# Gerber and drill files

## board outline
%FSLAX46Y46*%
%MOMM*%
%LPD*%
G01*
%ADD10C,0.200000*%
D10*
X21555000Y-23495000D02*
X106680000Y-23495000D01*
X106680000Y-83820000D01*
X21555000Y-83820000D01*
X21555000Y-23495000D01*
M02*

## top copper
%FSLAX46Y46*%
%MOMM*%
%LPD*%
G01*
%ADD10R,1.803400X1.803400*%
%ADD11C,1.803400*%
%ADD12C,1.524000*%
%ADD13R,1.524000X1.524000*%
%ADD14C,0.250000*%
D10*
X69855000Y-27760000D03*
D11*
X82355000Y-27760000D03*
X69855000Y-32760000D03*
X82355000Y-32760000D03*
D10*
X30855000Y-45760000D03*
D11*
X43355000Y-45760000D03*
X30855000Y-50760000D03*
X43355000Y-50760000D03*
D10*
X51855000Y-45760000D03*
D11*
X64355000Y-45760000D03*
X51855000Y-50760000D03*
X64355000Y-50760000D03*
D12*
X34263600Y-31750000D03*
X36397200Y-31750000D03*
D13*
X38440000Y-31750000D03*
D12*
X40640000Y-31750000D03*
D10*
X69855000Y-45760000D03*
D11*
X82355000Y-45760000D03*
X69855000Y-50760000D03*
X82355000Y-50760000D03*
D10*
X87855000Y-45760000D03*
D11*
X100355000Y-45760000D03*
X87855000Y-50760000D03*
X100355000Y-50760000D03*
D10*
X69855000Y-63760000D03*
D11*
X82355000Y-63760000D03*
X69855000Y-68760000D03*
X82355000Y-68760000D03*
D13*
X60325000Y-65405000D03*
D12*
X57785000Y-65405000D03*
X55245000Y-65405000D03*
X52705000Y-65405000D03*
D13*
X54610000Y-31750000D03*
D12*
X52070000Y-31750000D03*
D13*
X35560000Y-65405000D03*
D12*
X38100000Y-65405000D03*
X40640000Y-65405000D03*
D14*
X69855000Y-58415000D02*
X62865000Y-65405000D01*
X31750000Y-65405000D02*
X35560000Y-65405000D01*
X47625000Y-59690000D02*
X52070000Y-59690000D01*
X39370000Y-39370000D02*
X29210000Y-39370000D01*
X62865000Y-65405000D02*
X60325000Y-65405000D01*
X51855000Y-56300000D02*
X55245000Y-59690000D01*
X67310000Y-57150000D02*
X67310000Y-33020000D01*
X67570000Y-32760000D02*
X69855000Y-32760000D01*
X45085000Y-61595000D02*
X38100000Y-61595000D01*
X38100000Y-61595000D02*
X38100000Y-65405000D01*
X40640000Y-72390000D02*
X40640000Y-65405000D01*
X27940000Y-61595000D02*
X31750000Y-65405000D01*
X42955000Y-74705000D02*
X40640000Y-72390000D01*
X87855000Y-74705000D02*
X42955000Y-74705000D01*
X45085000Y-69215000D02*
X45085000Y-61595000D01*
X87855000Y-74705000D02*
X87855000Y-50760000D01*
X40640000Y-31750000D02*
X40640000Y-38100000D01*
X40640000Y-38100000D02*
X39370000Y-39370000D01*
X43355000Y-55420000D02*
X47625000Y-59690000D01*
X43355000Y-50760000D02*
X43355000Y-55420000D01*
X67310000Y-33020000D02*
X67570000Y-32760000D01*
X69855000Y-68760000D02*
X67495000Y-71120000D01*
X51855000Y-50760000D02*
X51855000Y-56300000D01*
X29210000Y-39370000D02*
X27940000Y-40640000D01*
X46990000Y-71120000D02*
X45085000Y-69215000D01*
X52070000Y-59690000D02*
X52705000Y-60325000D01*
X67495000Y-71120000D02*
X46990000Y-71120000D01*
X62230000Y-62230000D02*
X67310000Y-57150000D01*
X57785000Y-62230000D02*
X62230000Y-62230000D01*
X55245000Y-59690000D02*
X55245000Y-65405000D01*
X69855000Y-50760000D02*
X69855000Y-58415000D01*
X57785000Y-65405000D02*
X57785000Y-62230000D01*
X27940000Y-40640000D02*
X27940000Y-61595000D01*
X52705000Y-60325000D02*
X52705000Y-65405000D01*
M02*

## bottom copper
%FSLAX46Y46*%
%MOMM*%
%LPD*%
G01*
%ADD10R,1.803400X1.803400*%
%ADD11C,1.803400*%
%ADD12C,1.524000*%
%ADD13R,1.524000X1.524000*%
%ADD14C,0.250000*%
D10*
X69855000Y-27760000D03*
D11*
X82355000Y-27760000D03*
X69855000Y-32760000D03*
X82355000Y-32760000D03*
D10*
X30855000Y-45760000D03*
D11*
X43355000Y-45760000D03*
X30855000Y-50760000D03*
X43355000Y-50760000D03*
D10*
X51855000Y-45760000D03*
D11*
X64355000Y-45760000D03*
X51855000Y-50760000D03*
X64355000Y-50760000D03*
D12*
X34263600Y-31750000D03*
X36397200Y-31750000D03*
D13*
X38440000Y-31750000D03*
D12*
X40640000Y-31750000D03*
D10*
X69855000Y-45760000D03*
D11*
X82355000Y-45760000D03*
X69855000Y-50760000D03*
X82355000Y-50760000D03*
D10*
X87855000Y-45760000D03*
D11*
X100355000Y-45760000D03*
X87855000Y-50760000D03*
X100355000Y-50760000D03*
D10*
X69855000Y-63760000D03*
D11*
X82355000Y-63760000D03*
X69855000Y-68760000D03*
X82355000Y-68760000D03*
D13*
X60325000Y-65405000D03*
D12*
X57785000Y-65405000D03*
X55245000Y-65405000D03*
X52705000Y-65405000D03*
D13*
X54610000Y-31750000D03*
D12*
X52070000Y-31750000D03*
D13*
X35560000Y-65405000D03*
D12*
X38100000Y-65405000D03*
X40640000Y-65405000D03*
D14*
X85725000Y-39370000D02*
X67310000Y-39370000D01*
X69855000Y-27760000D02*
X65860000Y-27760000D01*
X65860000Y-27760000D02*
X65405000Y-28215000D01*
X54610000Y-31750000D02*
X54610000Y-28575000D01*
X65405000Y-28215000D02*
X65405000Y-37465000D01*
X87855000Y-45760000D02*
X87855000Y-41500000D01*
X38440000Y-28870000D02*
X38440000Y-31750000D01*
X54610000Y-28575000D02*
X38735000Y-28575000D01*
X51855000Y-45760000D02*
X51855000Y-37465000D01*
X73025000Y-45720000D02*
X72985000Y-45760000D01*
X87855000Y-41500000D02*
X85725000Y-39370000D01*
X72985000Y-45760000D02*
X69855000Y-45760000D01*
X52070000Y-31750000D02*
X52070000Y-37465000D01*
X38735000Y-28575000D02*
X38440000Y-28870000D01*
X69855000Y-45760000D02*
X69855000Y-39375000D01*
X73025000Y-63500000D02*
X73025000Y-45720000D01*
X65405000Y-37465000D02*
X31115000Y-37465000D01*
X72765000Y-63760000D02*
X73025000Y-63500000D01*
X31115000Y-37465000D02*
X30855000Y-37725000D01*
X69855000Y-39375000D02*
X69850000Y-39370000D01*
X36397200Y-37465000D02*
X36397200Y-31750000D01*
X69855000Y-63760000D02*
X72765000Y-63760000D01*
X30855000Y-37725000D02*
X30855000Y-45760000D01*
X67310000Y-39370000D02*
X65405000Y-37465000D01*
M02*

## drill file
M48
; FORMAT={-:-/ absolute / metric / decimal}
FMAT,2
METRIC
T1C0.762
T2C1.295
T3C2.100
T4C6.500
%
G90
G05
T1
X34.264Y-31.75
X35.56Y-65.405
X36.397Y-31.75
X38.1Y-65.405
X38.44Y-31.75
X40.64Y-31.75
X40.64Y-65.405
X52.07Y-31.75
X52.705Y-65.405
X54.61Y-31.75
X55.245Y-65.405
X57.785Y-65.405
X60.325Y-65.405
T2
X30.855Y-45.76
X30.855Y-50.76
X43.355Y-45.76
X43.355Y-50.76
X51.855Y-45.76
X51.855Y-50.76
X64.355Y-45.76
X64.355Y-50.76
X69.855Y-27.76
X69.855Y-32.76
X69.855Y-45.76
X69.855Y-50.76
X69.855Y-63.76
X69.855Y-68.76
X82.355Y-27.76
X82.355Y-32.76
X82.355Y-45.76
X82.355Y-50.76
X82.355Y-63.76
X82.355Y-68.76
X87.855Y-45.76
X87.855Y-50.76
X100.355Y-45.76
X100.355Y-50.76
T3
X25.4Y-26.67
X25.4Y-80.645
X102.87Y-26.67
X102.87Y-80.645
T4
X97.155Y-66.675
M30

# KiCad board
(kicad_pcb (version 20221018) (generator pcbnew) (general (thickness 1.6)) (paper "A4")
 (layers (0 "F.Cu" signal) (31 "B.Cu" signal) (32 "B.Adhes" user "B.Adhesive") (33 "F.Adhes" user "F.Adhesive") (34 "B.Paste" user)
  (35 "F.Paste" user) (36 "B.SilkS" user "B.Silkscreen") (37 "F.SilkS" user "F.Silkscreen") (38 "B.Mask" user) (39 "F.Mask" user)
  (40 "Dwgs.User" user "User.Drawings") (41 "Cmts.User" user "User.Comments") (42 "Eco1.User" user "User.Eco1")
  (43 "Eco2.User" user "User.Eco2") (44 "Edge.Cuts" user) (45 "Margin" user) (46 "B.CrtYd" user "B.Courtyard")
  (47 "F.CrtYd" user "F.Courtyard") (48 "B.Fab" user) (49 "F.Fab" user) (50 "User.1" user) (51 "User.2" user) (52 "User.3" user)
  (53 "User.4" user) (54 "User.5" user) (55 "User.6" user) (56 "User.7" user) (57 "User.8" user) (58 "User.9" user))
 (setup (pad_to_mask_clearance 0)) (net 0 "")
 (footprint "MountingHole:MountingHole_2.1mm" (layer "F.Cu") (at 102.87 80.645)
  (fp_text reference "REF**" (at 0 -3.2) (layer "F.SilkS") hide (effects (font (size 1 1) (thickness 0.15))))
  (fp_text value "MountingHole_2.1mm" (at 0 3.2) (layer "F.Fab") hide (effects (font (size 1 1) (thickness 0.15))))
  (pad "" np_thru_hole circle (at 0 0) (size 2.1 2.1) (drill 2.1) (layers "F&B.Cu" "*.Mask")))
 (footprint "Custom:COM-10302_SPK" (layer "F.Cu") (at 69.855 27.76)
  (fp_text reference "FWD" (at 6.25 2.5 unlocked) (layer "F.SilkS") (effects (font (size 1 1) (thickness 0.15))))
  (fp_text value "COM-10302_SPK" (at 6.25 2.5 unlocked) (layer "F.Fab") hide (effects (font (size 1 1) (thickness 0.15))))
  (pad "1" thru_hole rect (at 0 0) (size 1.8034 1.8034) (drill 1.2954) (layers "*.Cu" "*.Mask"))
  (pad "2" thru_hole circle (at 12.5 0) (size 1.8034 1.8034) (drill 1.2954) (layers "*.Cu" "*.Mask"))
  (pad "3" thru_hole circle (at 0 5) (size 1.8034 1.8034) (drill 1.2954) (layers "*.Cu" "*.Mask"))
  (pad "4" thru_hole circle (at 12.5 5) (size 1.8034 1.8034) (drill 1.2954) (layers "*.Cu" "*.Mask")))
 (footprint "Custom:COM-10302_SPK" (layer "F.Cu") (at 30.855 45.76)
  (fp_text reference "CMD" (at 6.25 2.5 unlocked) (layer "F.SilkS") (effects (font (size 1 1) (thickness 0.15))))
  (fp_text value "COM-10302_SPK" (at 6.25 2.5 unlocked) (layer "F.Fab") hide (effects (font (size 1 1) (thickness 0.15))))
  (pad "1" thru_hole rect (at 0 0) (size 1.8034 1.8034) (drill 1.2954) (layers "*.Cu" "*.Mask"))
  (pad "2" thru_hole circle (at 12.5 0) (size 1.8034 1.8034) (drill 1.2954) (layers "*.Cu" "*.Mask"))
  (pad "3" thru_hole circle (at 0 5) (size 1.8034 1.8034) (drill 1.2954) (layers "*.Cu" "*.Mask"))
  (pad "4" thru_hole circle (at 12.5 5) (size 1.8034 1.8034) (drill 1.2954) (layers "*.Cu" "*.Mask")))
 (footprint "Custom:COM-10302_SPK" (layer "F.Cu") (at 51.855 45.76)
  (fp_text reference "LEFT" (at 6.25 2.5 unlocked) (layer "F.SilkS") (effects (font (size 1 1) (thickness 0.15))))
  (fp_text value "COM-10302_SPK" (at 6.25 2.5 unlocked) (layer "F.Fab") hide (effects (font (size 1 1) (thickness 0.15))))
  (pad "1" thru_hole rect (at 0 0) (size 1.8034 1.8034) (drill 1.2954) (layers "*.Cu" "*.Mask"))
  (pad "2" thru_hole circle (at 12.5 0) (size 1.8034 1.8034) (drill 1.2954) (layers "*.Cu" "*.Mask"))
  (pad "3" thru_hole circle (at 0 5) (size 1.8034 1.8034) (drill 1.2954) (layers "*.Cu" "*.Mask"))
  (pad "4" thru_hole circle (at 12.5 5) (size 1.8034 1.8034) (drill 1.2954) (layers "*.Cu" "*.Mask")))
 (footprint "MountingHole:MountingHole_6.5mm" (layer "F.Cu") (at 97.155 66.675)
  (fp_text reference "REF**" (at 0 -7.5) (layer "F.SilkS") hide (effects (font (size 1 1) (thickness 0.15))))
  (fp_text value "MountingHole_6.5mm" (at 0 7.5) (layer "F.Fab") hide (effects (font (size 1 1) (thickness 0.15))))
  (pad "" np_thru_hole circle (at 0 0) (size 6.5 6.5) (drill 6.5) (layers "F&B.Cu" "*.Mask")))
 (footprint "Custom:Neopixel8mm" (layer "F.Cu") (at 35.94 31.75)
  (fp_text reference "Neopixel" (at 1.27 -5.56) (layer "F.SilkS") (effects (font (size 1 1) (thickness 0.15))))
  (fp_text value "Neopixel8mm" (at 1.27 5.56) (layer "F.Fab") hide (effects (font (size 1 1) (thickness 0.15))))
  (pad "1" thru_hole circle (at -1.6764 0) (size 1.524 1.524) (drill 0.762) (layers "*.Cu" "*.Mask"))
  (pad "2" thru_hole circle (at 0.4572 0) (size 1.524 1.524) (drill 0.762) (layers "*.Cu" "*.Mask"))
  (pad "3" thru_hole rect (at 2.5 0) (size 1.524 1.524) (drill 0.762) (layers "*.Cu" "*.Mask"))
  (pad "4" thru_hole circle (at 4.7 0) (size 1.524 1.524) (drill 0.762) (layers "*.Cu" "*.Mask")))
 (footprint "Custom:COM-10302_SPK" (layer "F.Cu") (at 69.855 45.76)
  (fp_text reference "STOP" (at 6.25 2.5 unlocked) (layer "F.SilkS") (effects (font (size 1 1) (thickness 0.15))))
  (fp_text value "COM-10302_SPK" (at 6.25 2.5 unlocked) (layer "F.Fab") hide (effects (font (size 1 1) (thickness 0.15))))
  (pad "1" thru_hole rect (at 0 0) (size 1.8034 1.8034) (drill 1.2954) (layers "*.Cu" "*.Mask"))
  (pad "2" thru_hole circle (at 12.5 0) (size 1.8034 1.8034) (drill 1.2954) (layers "*.Cu" "*.Mask"))
  (pad "3" thru_hole circle (at 0 5) (size 1.8034 1.8034) (drill 1.2954) (layers "*.Cu" "*.Mask"))
  (pad "4" thru_hole circle (at 12.5 5) (size 1.8034 1.8034) (drill 1.2954) (layers "*.Cu" "*.Mask")))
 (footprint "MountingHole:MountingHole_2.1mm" (layer "F.Cu") (at 102.87 26.67)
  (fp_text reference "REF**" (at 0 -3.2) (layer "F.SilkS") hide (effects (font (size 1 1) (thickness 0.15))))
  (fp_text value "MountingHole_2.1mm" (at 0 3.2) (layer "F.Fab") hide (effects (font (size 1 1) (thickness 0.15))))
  (pad "" np_thru_hole circle (at 0 0) (size 2.1 2.1) (drill 2.1) (layers "F&B.Cu" "*.Mask")))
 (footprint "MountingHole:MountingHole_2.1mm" (layer "F.Cu") (at 25.4 80.645)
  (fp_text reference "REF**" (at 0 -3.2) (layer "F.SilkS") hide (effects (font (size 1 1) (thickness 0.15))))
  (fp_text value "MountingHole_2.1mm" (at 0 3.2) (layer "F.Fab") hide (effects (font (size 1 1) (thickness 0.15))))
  (pad "" np_thru_hole circle (at 0 0) (size 2.1 2.1) (drill 2.1) (layers "F&B.Cu" "*.Mask")))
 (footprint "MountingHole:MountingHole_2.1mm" (layer "F.Cu") (at 25.4 26.67)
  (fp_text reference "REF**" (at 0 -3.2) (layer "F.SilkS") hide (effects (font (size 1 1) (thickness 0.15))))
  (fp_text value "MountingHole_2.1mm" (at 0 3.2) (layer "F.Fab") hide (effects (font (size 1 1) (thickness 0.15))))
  (pad "" np_thru_hole circle (at 0 0) (size 2.1 2.1) (drill 2.1) (layers "F&B.Cu" "*.Mask")))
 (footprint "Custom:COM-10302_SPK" (layer "F.Cu") (at 87.855 45.76)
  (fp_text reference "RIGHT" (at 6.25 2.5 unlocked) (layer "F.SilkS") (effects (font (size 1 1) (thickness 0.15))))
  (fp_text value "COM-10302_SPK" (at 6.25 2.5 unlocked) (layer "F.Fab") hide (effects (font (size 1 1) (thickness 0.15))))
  (pad "1" thru_hole rect (at 0 0) (size 1.8034 1.8034) (drill 1.2954) (layers "*.Cu" "*.Mask"))
  (pad "2" thru_hole circle (at 12.5 0) (size 1.8034 1.8034) (drill 1.2954) (layers "*.Cu" "*.Mask"))
  (pad "3" thru_hole circle (at 0 5) (size 1.8034 1.8034) (drill 1.2954) (layers "*.Cu" "*.Mask"))
  (pad "4" thru_hole circle (at 12.5 5) (size 1.8034 1.8034) (drill 1.2954) (layers "*.Cu" "*.Mask")))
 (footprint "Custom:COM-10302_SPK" (layer "F.Cu") (at 69.855 63.76)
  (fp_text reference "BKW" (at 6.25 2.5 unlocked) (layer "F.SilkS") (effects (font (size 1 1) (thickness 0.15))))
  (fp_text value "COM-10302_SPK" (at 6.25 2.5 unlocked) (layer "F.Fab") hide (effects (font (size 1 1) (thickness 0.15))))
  (pad "1" thru_hole rect (at 0 0) (size 1.8034 1.8034) (drill 1.2954) (layers "*.Cu" "*.Mask"))
  (pad "2" thru_hole circle (at 12.5 0) (size 1.8034 1.8034) (drill 1.2954) (layers "*.Cu" "*.Mask"))
  (pad "3" thru_hole circle (at 0 5) (size 1.8034 1.8034) (drill 1.2954) (layers "*.Cu" "*.Mask"))
  (pad "4" thru_hole circle (at 12.5 5) (size 1.8034 1.8034) (drill 1.2954) (layers "*.Cu" "*.Mask")))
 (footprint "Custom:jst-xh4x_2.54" (layer "B.Cu") (at 55.245 67.945 90)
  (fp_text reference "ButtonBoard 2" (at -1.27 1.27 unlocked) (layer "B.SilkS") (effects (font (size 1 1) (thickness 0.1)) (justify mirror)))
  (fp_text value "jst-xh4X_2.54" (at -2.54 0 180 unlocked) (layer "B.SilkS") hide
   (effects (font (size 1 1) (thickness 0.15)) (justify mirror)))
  (pad "1" thru_hole rect (at 2.54 5.08 90) (size 1.524 1.524) (drill 0.762) (layers "*.Cu" "*.Mask"))
  (pad "2" thru_hole circle (at 2.54 2.54 90) (size 1.524 1.524) (drill 0.762) (layers "*.Cu" "*.Mask"))
  (pad "3" thru_hole circle (at 2.54 0 90) (size 1.524 1.524) (drill 0.762) (layers "*.Cu" "*.Mask"))
  (pad "4" thru_hole circle (at 2.54 -2.54 90) (size 1.524 1.524) (drill 0.762) (layers "*.Cu" "*.Mask")))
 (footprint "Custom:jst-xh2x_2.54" (layer "B.Cu") (at 53.34 31.75 90)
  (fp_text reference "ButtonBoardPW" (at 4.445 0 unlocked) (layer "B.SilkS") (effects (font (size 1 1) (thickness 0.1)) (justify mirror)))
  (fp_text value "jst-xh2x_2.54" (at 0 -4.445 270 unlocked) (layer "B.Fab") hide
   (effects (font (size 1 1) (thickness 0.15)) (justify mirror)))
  (pad "1" thru_hole rect (at 0 1.27 90) (size 1.524 1.524) (drill 0.762) (layers "*.Cu" "*.Mask"))
  (pad "2" thru_hole circle (at 0 -1.27 90) (size 1.524 1.524) (drill 0.762) (layers "*.Cu" "*.Mask")))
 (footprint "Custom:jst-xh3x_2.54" (layer "B.Cu") (at 40.64 62.865 -90)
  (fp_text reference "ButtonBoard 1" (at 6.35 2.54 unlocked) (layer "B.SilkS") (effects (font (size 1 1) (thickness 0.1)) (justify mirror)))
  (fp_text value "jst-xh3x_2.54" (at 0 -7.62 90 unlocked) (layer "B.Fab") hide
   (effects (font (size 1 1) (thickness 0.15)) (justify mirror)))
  (pad "1" thru_hole rect (at 2.54 5.08 270) (size 1.524 1.524) (drill 0.762) (layers "*.Cu" "*.Mask"))
  (pad "2" thru_hole circle (at 2.54 2.54 270) (size 1.524 1.524) (drill 0.762) (layers "*.Cu" "*.Mask"))
  (pad "3" thru_hole circle (at 2.54 0 270) (size 1.524 1.524) (drill 0.762) (layers "*.Cu" "*.Mask")))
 (gr_rect (start 112.395 26.035) (end 112.395 26.035) (stroke (width 0.2) (type default)) (fill none) (layer "F.Cu"))
 (gr_rect (start 21.555 23.495) (end 106.68 83.82) (stroke (width 0.2) (type default)) (fill none) (layer "Edge.Cuts"))
 (segment (start 69.855 58.415) (end 62.865 65.405) (width 0.25) (layer "F.Cu") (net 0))
 (segment (start 31.75 65.405) (end 35.56 65.405) (width 0.25) (layer "F.Cu") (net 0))
 (segment (start 47.625 59.69) (end 52.07 59.69) (width 0.25) (layer "F.Cu") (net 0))
 (segment (start 39.37 39.37) (end 29.21 39.37) (width 0.25) (layer "F.Cu") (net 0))
 (segment (start 62.865 65.405) (end 60.325 65.405) (width 0.25) (layer "F.Cu") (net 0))
 (segment (start 51.855 56.3) (end 55.245 59.69) (width 0.25) (layer "F.Cu") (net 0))
 (segment (start 67.31 57.15) (end 67.31 33.02) (width 0.25) (layer "F.Cu") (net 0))
 (segment (start 67.57 32.76) (end 69.855 32.76) (width 0.25) (layer "F.Cu") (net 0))
 (segment (start 45.085 61.595) (end 38.1 61.595) (width 0.25) (layer "F.Cu") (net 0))
 (segment (start 38.1 61.595) (end 38.1 65.405) (width 0.25) (layer "F.Cu") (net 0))
 (segment (start 40.64 72.39) (end 40.64 65.405) (width 0.25) (layer "F.Cu") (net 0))
 (segment (start 27.94 61.595) (end 31.75 65.405) (width 0.25) (layer "F.Cu") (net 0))
 (segment (start 42.955 74.705) (end 40.64 72.39) (width 0.25) (layer "F.Cu") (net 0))
 (segment (start 87.855 74.705) (end 42.955 74.705) (width 0.25) (layer "F.Cu") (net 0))
 (segment (start 45.085 69.215) (end 45.085 61.595) (width 0.25) (layer "F.Cu") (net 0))
 (segment (start 87.855 74.705) (end 87.855 50.76) (width 0.25) (layer "F.Cu") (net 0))
 (segment (start 40.64 31.75) (end 40.64 38.1) (width 0.25) (layer "F.Cu") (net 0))
 (segment (start 40.64 38.1) (end 39.37 39.37) (width 0.25) (layer "F.Cu") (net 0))
 (segment (start 43.355 55.42) (end 47.625 59.69) (width 0.25) (layer "F.Cu") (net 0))
 (segment (start 43.355 50.76) (end 43.355 55.42) (width 0.25) (layer "F.Cu") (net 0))
 (segment (start 67.31 33.02) (end 67.57 32.76) (width 0.25) (layer "F.Cu") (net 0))
 (segment (start 69.855 68.76) (end 67.495 71.12) (width 0.25) (layer "F.Cu") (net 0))
 (segment (start 51.855 50.76) (end 51.855 56.3) (width 0.25) (layer "F.Cu") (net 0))
 (segment (start 29.21 39.37) (end 27.94 40.64) (width 0.25) (layer "F.Cu") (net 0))
 (segment (start 46.99 71.12) (end 45.085 69.215) (width 0.25) (layer "F.Cu") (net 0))
 (segment (start 52.07 59.69) (end 52.705 60.325) (width 0.25) (layer "F.Cu") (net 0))
 (segment (start 67.495 71.12) (end 46.99 71.12) (width 0.25) (layer "F.Cu") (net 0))
 (segment (start 62.23 62.23) (end 67.31 57.15) (width 0.25) (layer "F.Cu") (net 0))
 (segment (start 57.785 62.23) (end 62.23 62.23) (width 0.25) (layer "F.Cu") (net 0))
 (segment (start 55.245 59.69) (end 55.245 65.405) (width 0.25) (layer "F.Cu") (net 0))
 (segment (start 69.855 50.76) (end 69.855 58.415) (width 0.25) (layer "F.Cu") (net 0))
 (segment (start 57.785 65.405) (end 57.785 62.23) (width 0.25) (layer "F.Cu") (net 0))
 (segment (start 27.94 40.64) (end 27.94 61.595) (width 0.25) (layer "F.Cu") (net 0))
 (segment (start 52.705 60.325) (end 52.705 65.405) (width 0.25) (layer "F.Cu") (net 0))
 (segment (start 85.725 39.37) (end 67.31 39.37) (width 0.25) (layer "B.Cu") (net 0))
 (segment (start 69.855 27.76) (end 65.86 27.76) (width 0.25) (layer "B.Cu") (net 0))
 (segment (start 65.86 27.76) (end 65.405 28.215) (width 0.25) (layer "B.Cu") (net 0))
 (segment (start 54.61 31.75) (end 54.61 28.575) (width 0.25) (layer "B.Cu") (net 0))
 (segment (start 65.405 28.215) (end 65.405 37.465) (width 0.25) (layer "B.Cu") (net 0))
 (segment (start 87.855 45.76) (end 87.855 41.5) (width 0.25) (layer "B.Cu") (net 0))
 (segment (start 38.44 28.87) (end 38.44 31.75) (width 0.25) (layer "B.Cu") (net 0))
 (segment (start 54.61 28.575) (end 38.735 28.575) (width 0.25) (layer "B.Cu") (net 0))
 (segment (start 51.855 45.76) (end 51.855 37.465) (width 0.25) (layer "B.Cu") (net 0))
 (segment (start 73.025 45.72) (end 72.985 45.76) (width 0.25) (layer "B.Cu") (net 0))
 (segment (start 87.855 41.5) (end 85.725 39.37) (width 0.25) (layer "B.Cu") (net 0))
 (segment (start 72.985 45.76) (end 69.855 45.76) (width 0.25) (layer "B.Cu") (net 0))
 (segment (start 52.07 31.75) (end 52.07 37.465) (width 0.25) (layer "B.Cu") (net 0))
 (segment (start 38.735 28.575) (end 38.44 28.87) (width 0.25) (layer "B.Cu") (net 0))
 (segment (start 69.855 45.76) (end 69.855 39.375) (width 0.25) (layer "B.Cu") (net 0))
 (segment (start 73.025 63.5) (end 73.025 45.72) (width 0.25) (layer "B.Cu") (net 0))
 (segment (start 65.405 37.465) (end 31.115 37.465) (width 0.25) (layer "B.Cu") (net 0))
 (segment (start 72.765 63.76) (end 73.025 63.5) (width 0.25) (layer "B.Cu") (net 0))
 (segment (start 31.115 37.465) (end 30.855 37.725) (width 0.25) (layer "B.Cu") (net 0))
 (segment (start 69.855 39.375) (end 69.85 39.37) (width 0.25) (layer "B.Cu") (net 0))
 (segment (start 36.3972 37.465) (end 36.3972 31.75) (width 0.25) (layer "B.Cu") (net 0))
 (segment (start 69.855 63.76) (end 72.765 63.76) (width 0.25) (layer "B.Cu") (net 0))
 (segment (start 30.855 37.725) (end 30.855 45.76) (width 0.25) (layer "B.Cu") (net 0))
 (segment (start 67.31 39.37) (end 65.405 37.465) (width 0.25) (layer "B.Cu") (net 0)))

